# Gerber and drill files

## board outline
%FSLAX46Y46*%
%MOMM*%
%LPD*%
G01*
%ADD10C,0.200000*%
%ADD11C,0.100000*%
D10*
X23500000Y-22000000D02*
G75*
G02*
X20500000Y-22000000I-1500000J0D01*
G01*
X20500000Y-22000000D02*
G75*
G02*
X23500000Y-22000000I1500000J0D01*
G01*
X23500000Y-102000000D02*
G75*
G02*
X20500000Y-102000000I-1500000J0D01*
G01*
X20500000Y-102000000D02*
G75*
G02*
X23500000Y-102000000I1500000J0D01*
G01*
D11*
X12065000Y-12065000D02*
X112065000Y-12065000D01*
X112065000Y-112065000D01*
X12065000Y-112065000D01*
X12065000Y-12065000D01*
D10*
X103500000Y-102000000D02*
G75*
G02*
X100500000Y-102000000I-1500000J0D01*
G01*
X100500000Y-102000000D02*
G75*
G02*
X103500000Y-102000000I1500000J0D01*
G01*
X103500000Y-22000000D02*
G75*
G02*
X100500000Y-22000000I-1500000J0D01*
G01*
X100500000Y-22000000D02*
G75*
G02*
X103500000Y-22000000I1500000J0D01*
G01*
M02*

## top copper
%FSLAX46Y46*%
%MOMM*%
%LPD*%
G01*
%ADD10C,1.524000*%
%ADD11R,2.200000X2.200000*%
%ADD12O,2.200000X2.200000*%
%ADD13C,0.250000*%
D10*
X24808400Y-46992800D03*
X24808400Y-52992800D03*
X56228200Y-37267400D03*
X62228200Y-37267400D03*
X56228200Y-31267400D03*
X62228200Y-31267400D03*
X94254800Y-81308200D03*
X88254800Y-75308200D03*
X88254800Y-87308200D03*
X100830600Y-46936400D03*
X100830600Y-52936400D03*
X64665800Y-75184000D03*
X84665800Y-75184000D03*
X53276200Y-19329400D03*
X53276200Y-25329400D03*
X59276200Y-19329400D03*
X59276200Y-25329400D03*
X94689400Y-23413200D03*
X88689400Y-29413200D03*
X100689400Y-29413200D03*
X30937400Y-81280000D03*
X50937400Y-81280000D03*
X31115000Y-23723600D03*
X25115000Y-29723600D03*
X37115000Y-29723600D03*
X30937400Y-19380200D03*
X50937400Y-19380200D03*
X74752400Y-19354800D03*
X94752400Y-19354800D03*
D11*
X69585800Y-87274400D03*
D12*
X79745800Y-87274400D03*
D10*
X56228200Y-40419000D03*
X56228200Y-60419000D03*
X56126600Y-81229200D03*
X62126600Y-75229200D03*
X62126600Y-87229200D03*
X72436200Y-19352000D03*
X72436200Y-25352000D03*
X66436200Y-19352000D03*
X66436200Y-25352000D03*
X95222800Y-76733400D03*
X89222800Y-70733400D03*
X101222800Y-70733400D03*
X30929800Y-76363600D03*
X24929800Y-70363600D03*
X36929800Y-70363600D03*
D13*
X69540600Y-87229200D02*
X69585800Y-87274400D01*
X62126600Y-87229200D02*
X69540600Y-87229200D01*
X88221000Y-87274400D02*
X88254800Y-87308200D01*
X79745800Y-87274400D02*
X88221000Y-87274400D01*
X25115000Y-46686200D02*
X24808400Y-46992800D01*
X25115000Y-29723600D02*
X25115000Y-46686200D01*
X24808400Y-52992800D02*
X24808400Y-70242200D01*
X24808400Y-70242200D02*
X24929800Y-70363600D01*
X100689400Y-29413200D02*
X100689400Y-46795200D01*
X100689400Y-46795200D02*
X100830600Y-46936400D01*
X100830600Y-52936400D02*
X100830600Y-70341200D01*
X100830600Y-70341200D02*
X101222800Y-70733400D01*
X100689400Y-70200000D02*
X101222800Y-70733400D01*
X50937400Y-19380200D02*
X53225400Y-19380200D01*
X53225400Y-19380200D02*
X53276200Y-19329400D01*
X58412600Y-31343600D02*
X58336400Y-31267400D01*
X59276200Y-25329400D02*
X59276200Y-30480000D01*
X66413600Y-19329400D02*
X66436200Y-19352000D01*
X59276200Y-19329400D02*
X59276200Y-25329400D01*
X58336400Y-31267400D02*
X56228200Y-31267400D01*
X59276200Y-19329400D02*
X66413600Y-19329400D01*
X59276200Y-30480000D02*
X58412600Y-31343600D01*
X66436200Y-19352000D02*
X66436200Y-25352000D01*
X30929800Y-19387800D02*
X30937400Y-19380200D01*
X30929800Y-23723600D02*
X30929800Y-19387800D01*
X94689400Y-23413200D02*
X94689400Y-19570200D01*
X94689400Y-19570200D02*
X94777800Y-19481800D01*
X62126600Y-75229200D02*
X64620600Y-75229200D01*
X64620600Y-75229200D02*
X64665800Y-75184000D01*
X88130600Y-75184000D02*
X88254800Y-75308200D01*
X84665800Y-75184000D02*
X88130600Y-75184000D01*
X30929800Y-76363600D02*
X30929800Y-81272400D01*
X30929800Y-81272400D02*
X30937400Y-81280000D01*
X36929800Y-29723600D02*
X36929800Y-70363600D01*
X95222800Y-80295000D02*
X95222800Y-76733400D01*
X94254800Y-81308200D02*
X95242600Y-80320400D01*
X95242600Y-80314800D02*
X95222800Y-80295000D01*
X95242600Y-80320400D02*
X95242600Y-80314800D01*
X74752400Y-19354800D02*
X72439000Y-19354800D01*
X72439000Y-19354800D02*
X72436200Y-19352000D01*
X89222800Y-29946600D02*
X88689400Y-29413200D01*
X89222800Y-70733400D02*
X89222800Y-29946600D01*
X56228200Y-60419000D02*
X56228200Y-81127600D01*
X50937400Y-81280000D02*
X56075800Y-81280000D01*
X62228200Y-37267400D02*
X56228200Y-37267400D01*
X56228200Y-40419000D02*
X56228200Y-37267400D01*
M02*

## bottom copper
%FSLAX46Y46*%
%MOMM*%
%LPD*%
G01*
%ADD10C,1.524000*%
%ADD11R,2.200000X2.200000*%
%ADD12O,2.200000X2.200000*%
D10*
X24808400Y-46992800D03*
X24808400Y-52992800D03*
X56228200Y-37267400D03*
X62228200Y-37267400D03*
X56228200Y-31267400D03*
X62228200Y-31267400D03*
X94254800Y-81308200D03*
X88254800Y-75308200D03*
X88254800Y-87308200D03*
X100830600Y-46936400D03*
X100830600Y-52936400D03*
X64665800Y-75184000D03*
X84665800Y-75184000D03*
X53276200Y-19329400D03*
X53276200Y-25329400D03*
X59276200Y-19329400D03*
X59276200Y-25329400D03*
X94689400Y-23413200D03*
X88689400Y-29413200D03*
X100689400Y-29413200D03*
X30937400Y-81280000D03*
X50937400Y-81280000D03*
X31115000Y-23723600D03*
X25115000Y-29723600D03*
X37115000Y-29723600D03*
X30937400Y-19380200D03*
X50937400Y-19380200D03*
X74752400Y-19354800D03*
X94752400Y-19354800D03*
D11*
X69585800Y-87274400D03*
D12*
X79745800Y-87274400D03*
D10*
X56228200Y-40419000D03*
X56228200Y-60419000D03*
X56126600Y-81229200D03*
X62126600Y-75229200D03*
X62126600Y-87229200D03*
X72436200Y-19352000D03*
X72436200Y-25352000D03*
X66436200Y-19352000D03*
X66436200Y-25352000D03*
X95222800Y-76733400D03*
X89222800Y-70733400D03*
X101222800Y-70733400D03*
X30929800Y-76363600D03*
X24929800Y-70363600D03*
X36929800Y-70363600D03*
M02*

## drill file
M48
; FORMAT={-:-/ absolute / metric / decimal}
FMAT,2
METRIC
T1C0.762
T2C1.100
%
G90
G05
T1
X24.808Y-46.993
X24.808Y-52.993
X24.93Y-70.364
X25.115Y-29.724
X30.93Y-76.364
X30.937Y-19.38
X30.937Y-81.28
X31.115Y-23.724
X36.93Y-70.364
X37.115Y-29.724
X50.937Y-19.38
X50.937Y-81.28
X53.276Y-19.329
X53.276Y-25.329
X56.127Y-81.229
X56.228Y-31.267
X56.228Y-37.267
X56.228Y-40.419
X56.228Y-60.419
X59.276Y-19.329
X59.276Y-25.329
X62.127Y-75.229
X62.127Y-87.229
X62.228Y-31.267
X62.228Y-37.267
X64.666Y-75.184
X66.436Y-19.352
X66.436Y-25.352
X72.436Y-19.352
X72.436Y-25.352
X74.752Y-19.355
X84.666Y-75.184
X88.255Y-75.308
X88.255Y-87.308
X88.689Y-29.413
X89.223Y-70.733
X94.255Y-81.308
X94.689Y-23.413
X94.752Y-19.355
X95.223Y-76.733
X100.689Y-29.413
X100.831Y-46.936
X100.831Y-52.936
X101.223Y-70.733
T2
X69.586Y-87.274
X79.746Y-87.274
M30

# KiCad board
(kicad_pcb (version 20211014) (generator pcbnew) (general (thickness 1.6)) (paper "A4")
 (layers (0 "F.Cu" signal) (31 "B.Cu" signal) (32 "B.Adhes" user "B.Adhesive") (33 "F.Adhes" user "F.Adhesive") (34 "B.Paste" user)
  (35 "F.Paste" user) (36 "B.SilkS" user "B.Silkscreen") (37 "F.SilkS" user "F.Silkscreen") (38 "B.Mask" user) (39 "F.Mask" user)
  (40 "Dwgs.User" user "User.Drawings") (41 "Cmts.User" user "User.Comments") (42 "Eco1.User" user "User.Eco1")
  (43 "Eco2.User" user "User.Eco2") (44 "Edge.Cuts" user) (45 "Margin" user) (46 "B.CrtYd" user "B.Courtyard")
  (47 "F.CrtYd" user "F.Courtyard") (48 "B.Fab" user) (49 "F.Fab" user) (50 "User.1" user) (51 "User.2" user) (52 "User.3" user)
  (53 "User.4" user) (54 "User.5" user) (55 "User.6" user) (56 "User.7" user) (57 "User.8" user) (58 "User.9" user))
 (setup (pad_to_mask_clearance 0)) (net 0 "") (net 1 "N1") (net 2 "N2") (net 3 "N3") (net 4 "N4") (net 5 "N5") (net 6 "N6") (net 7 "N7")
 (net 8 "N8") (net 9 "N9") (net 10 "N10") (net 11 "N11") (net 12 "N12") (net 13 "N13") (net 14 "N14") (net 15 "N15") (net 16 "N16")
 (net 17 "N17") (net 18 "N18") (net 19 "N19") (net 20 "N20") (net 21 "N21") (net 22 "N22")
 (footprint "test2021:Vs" (layer "F.Cu") (at 24.8084 49.9928)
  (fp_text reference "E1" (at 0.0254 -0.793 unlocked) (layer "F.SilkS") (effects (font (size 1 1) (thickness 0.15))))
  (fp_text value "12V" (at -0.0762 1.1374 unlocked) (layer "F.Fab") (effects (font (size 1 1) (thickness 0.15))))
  (pad "1" thru_hole circle (at 0 -3) (size 1.524 1.524) (drill 0.762) (layers *.Cu *.Mask) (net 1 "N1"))
  (pad "2" thru_hole circle (at 0 3) (size 1.524 1.524) (drill 0.762) (layers *.Cu *.Mask) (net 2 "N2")))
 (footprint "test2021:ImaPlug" (layer "F.Cu") (at 59.2282 34.2674 90)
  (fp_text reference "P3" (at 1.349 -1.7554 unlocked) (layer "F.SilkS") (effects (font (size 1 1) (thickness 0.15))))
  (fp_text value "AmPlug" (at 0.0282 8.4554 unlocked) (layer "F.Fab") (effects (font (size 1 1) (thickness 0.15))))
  (pad "1" thru_hole circle (at -3 -3 90) (size 1.524 1.524) (drill 0.762) (layers *.Cu *.Mask) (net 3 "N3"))
  (pad "2" thru_hole circle (at -3 3 90) (size 1.524 1.524) (drill 0.762) (layers *.Cu *.Mask) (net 3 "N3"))
  (pad "3" thru_hole circle (at 3 -3 90) (size 1.524 1.524) (drill 0.762) (layers *.Cu *.Mask) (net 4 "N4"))
  (pad "4" thru_hole circle (at 3 3 90) (size 1.524 1.524) (drill 0.762) (layers *.Cu *.Mask) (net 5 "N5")))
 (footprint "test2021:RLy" (layer "F.Cu") (at 88.2548 81.3082 -90)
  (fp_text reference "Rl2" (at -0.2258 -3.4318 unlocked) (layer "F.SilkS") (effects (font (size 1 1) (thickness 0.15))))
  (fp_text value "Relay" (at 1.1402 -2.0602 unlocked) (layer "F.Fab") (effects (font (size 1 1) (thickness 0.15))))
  (pad "1" thru_hole circle (at 0 -6 270) (size 1.524 1.524) (drill 0.762) (layers *.Cu *.Mask) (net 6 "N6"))
  (pad "2" thru_hole circle (at -6 0 270) (size 1.524 1.524) (drill 0.762) (layers *.Cu *.Mask) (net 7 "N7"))
  (pad "3" thru_hole circle (at 6 0 270) (size 1.524 1.524) (drill 0.762) (layers *.Cu *.Mask) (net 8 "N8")))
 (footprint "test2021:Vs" (layer "F.Cu") (at 100.8306 49.9364)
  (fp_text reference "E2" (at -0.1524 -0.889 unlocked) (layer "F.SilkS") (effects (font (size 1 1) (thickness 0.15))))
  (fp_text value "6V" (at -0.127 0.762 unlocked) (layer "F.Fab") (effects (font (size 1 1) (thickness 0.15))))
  (pad "1" thru_hole circle (at 0 -3) (size 1.524 1.524) (drill 0.762) (layers *.Cu *.Mask) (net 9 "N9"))
  (pad "2" thru_hole circle (at 0 3) (size 1.524 1.524) (drill 0.762) (layers *.Cu *.Mask) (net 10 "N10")))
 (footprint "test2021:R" (layer "F.Cu") (at 74.6658 75.184)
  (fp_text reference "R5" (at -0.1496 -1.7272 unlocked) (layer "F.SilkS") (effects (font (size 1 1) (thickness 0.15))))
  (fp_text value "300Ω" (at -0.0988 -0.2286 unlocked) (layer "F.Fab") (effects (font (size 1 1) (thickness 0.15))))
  (pad "1" thru_hole circle (at -10 0) (size 1.524 1.524) (drill 0.762) (layers *.Cu *.Mask) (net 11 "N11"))
  (pad "2" thru_hole circle (at 10 0) (size 1.524 1.524) (drill 0.762) (layers *.Cu *.Mask) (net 7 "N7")))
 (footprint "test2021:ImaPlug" (layer "F.Cu") (at 56.2762 22.3294)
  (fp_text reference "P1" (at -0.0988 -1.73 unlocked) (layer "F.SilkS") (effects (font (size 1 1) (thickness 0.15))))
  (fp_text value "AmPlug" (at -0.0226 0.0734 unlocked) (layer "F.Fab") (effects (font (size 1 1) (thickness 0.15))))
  (pad "1" thru_hole circle (at -3 -3) (size 1.524 1.524) (drill 0.762) (layers *.Cu *.Mask) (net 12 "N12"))
  (pad "2" thru_hole circle (at -3 3) (size 1.524 1.524) (drill 0.762) (layers *.Cu *.Mask) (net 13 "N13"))
  (pad "3" thru_hole circle (at 3 -3) (size 1.524 1.524) (drill 0.762) (layers *.Cu *.Mask) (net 4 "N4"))
  (pad "4" thru_hole circle (at 3 3) (size 1.524 1.524) (drill 0.762) (layers *.Cu *.Mask) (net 4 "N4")))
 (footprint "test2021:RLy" (layer "F.Cu") (at 94.6894 29.4132)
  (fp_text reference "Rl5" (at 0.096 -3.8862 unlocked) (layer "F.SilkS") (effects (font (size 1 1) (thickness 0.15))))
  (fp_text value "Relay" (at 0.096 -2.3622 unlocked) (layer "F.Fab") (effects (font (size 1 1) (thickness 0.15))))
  (pad "1" thru_hole circle (at 0 -6) (size 1.524 1.524) (drill 0.762) (layers *.Cu *.Mask) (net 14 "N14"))
  (pad "2" thru_hole circle (at -6 0) (size 1.524 1.524) (drill 0.762) (layers *.Cu *.Mask) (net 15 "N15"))
  (pad "3" thru_hole circle (at 6 0) (size 1.524 1.524) (drill 0.762) (layers *.Cu *.Mask) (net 9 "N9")))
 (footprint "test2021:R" (layer "F.Cu") (at 40.9374 81.28)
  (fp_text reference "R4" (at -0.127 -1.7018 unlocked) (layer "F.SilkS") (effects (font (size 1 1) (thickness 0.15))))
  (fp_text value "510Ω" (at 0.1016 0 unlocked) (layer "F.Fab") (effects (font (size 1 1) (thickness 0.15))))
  (pad "1" thru_hole circle (at -10 0) (size 1.524 1.524) (drill 0.762) (layers *.Cu *.Mask) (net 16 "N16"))
  (pad "2" thru_hole circle (at 10 0) (size 1.524 1.524) (drill 0.762) (layers *.Cu *.Mask) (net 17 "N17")))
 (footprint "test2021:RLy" (layer "F.Cu") (at 31.115 29.7236)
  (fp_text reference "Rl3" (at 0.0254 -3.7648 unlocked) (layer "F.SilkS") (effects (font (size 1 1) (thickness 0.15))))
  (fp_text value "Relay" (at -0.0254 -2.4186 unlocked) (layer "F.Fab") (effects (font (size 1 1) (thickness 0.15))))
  (pad "1" thru_hole circle (at 0 -6) (size 1.524 1.524) (drill 0.762) (layers *.Cu *.Mask) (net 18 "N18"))
  (pad "2" thru_hole circle (at -6 0) (size 1.524 1.524) (drill 0.762) (layers *.Cu *.Mask) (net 1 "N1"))
  (pad "3" thru_hole circle (at 6 0) (size 1.524 1.524) (drill 0.762) (layers *.Cu *.Mask) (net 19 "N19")))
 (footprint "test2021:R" (layer "F.Cu") (at 40.9374 19.3802)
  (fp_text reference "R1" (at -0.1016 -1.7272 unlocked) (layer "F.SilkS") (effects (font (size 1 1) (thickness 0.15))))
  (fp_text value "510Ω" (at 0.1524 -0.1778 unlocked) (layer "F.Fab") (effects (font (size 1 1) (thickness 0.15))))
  (pad "1" thru_hole circle (at -10 0) (size 1.524 1.524) (drill 0.762) (layers *.Cu *.Mask) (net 18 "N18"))
  (pad "2" thru_hole circle (at 10 0) (size 1.524 1.524) (drill 0.762) (layers *.Cu *.Mask) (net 12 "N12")))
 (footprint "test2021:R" (layer "F.Cu") (at 84.7524 19.3548)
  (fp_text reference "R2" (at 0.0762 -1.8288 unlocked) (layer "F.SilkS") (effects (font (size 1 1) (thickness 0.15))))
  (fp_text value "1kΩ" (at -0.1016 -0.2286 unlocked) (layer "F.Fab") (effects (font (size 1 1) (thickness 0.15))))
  (pad "1" thru_hole circle (at -10 0) (size 1.524 1.524) (drill 0.762) (layers *.Cu *.Mask) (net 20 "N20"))
  (pad "2" thru_hole circle (at 10 0) (size 1.524 1.524) (drill 0.762) (layers *.Cu *.Mask) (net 14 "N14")))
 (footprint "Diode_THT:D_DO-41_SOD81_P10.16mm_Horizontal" (layer "F.Cu") (at 69.5858 87.2744)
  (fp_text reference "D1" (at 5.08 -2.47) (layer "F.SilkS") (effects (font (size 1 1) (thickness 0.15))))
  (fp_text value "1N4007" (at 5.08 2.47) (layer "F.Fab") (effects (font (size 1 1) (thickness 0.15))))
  (pad "1" thru_hole rect (at 0 0) (size 2.2 2.2) (drill 1.1) (layers *.Cu *.Mask) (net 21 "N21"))
  (pad "2" thru_hole oval (at 10.16 0) (size 2.2 2.2) (drill 1.1) (layers *.Cu *.Mask) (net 8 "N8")))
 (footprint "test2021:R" (layer "F.Cu") (at 56.2282 50.419 -90)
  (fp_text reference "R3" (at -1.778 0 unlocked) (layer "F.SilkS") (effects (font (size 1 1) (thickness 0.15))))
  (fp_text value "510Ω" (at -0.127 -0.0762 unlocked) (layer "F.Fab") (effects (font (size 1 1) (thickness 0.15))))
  (pad "1" thru_hole circle (at -10 0 270) (size 1.524 1.524) (drill 0.762) (layers *.Cu *.Mask) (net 3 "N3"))
  (pad "2" thru_hole circle (at 10 0 270) (size 1.524 1.524) (drill 0.762) (layers *.Cu *.Mask) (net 17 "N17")))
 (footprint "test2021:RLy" (layer "B.Cu") (at 62.1266 81.2292 -90)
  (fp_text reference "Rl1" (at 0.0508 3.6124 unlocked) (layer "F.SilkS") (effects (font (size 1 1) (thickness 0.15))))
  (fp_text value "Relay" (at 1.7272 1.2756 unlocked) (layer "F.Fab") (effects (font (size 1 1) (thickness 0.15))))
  (pad "1" thru_hole circle (at 0 6 270) (size 1.524 1.524) (drill 0.762) (layers *.Cu *.Mask) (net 17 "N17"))
  (pad "2" thru_hole circle (at -6 0 270) (size 1.524 1.524) (drill 0.762) (layers *.Cu *.Mask) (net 11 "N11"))
  (pad "3" thru_hole circle (at 6 0 270) (size 1.524 1.524) (drill 0.762) (layers *.Cu *.Mask) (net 21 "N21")))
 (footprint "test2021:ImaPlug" (layer "B.Cu") (at 69.4362 22.352 180)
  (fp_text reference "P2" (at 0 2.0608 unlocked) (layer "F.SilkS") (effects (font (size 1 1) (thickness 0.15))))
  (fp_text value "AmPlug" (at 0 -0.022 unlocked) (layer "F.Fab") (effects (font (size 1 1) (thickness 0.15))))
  (pad "1" thru_hole circle (at -3 3 180) (size 1.524 1.524) (drill 0.762) (layers *.Cu *.Mask) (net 20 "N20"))
  (pad "2" thru_hole circle (at -3 -3 180) (size 1.524 1.524) (drill 0.762) (layers *.Cu *.Mask) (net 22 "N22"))
  (pad "3" thru_hole circle (at 3 3 180) (size 1.524 1.524) (drill 0.762) (layers *.Cu *.Mask) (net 4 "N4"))
  (pad "4" thru_hole circle (at 3 -3 180) (size 1.524 1.524) (drill 0.762) (layers *.Cu *.Mask) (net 4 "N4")))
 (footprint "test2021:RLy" (layer "B.Cu") (at 95.2228 70.7334)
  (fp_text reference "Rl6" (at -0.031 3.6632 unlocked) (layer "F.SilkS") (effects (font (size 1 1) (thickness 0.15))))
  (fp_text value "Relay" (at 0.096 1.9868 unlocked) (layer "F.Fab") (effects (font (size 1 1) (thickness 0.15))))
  (pad "1" thru_hole circle (at 0 6) (size 1.524 1.524) (drill 0.762) (layers *.Cu *.Mask) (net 6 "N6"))
  (pad "2" thru_hole circle (at -6 0) (size 1.524 1.524) (drill 0.762) (layers *.Cu *.Mask) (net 15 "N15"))
  (pad "3" thru_hole circle (at 6 0) (size 1.524 1.524) (drill 0.762) (layers *.Cu *.Mask) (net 10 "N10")))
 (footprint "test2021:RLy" (layer "B.Cu") (at 30.9298 70.3636)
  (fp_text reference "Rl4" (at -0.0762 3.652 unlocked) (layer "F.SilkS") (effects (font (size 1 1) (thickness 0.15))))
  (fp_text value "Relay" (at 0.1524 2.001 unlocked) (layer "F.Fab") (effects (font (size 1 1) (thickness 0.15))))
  (pad "1" thru_hole circle (at 0 6) (size 1.524 1.524) (drill 0.762) (layers *.Cu *.Mask) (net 16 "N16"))
  (pad "2" thru_hole circle (at -6 0) (size 1.524 1.524) (drill 0.762) (layers *.Cu *.Mask) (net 2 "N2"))
  (pad "3" thru_hole circle (at 6 0) (size 1.524 1.524) (drill 0.762) (layers *.Cu *.Mask) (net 19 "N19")))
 (gr_circle (center 22 22) (end 23.5 22) (layer "Edge.Cuts") (width 0.2) (fill none))
 (gr_circle (center 22 102) (end 23.5 102) (layer "Edge.Cuts") (width 0.2) (fill none))
 (gr_rect (start 12.065 12.065) (end 112.065 112.065) (layer "Edge.Cuts") (width 0.1) (fill none))
 (gr_circle (center 102 102) (end 103.5 102) (layer "Edge.Cuts") (width 0.2) (fill none))
 (gr_circle (center 102 22) (end 103.5 22) (layer "Edge.Cuts") (width 0.2) (fill none))
 (segment (start 69.5406 87.2292) (end 69.5858 87.2744) (width 0.25) (layer "F.Cu") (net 21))
 (segment (start 62.1266 87.2292) (end 69.5406 87.2292) (width 0.25) (layer "F.Cu") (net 21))
 (segment (start 88.221 87.2744) (end 88.2548 87.3082) (width 0.25) (layer "F.Cu") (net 8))
 (segment (start 79.7458 87.2744) (end 88.221 87.2744) (width 0.25) (layer "F.Cu") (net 8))
 (segment (start 25.115 46.6862) (end 24.8084 46.9928) (width 0.25) (layer "F.Cu") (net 1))
 (segment (start 25.115 29.7236) (end 25.115 46.6862) (width 0.25) (layer "F.Cu") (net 1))
 (segment (start 24.8084 52.9928) (end 24.8084 70.2422) (width 0.25) (layer "F.Cu") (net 2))
 (segment (start 24.8084 70.2422) (end 24.9298 70.3636) (width 0.25) (layer "F.Cu") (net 2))
 (segment (start 100.6894 29.4132) (end 100.6894 46.7952) (width 0.25) (layer "F.Cu") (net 9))
 (segment (start 100.6894 46.7952) (end 100.8306 46.9364) (width 0.25) (layer "F.Cu") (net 9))
 (segment (start 100.8306 52.9364) (end 100.8306 70.3412) (width 0.25) (layer "F.Cu") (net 10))
 (segment (start 100.8306 70.3412) (end 101.2228 70.7334) (width 0.25) (layer "F.Cu") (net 10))
 (segment (start 100.6894 70.2) (end 101.2228 70.7334) (width 0.25) (layer "F.Cu") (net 10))
 (segment (start 50.9374 19.3802) (end 53.2254 19.3802) (width 0.25) (layer "F.Cu") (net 12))
 (segment (start 53.2254 19.3802) (end 53.2762 19.3294) (width 0.25) (layer "F.Cu") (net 12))
 (segment (start 58.4126 31.3436) (end 58.3364 31.2674) (width 0.25) (layer "F.Cu") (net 4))
 (segment (start 59.2762 25.3294) (end 59.2762 30.48) (width 0.25) (layer "F.Cu") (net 4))
 (segment (start 66.4136 19.3294) (end 66.4362 19.352) (width 0.25) (layer "F.Cu") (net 4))
 (segment (start 59.2762 19.3294) (end 59.2762 25.3294) (width 0.25) (layer "F.Cu") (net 4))
 (segment (start 58.3364 31.2674) (end 56.2282 31.2674) (width 0.25) (layer "F.Cu") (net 4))
 (segment (start 59.2762 19.3294) (end 66.4136 19.3294) (width 0.25) (layer "F.Cu") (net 4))
 (segment (start 59.2762 30.48) (end 58.4126 31.3436) (width 0.25) (layer "F.Cu") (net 4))
 (segment (start 66.4362 19.352) (end 66.4362 25.352) (width 0.25) (layer "F.Cu") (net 4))
 (segment (start 30.9298 19.3878) (end 30.9374 19.3802) (width 0.25) (layer "F.Cu") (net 18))
 (segment (start 30.9298 23.7236) (end 30.9298 19.3878) (width 0.25) (layer "F.Cu") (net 18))
 (segment (start 94.6894 23.4132) (end 94.6894 19.5702) (width 0.25) (layer "F.Cu") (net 14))
 (segment (start 94.6894 19.5702) (end 94.7778 19.4818) (width 0.25) (layer "F.Cu") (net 14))
 (segment (start 62.1266 75.2292) (end 64.6206 75.2292) (width 0.25) (layer "F.Cu") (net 11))
 (segment (start 64.6206 75.2292) (end 64.6658 75.184) (width 0.25) (layer "F.Cu") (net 11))
 (segment (start 88.1306 75.184) (end 88.2548 75.3082) (width 0.25) (layer "F.Cu") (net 7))
 (segment (start 84.6658 75.184) (end 88.1306 75.184) (width 0.25) (layer "F.Cu") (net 7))
 (segment (start 30.9298 76.3636) (end 30.9298 81.2724) (width 0.25) (layer "F.Cu") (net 16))
 (segment (start 30.9298 81.2724) (end 30.9374 81.28) (width 0.25) (layer "F.Cu") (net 16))
 (segment (start 36.9298 29.7236) (end 36.9298 70.3636) (width 0.25) (layer "F.Cu") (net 19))
 (segment (start 95.2228 80.295) (end 95.2228 76.7334) (width 0.25) (layer "F.Cu") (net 6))
 (segment (start 94.2548 81.3082) (end 95.2426 80.3204) (width 0.25) (layer "F.Cu") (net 6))
 (segment (start 95.2426 80.3148) (end 95.2228 80.295) (width 0.25) (layer "F.Cu") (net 6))
 (segment (start 95.2426 80.3204) (end 95.2426 80.3148) (width 0.25) (layer "F.Cu") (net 6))
 (segment (start 74.7524 19.3548) (end 72.439 19.3548) (width 0.25) (layer "F.Cu") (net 20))
 (segment (start 72.439 19.3548) (end 72.4362 19.352) (width 0.25) (layer "F.Cu") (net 20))
 (segment (start 89.2228 29.9466) (end 88.6894 29.4132) (width 0.25) (layer "F.Cu") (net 15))
 (segment (start 89.2228 70.7334) (end 89.2228 29.9466) (width 0.25) (layer "F.Cu") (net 15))
 (segment (start 56.2282 60.419) (end 56.2282 81.1276) (width 0.25) (layer "F.Cu") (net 17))
 (segment (start 50.9374 81.28) (end 56.0758 81.28) (width 0.25) (layer "F.Cu") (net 17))
 (segment (start 62.2282 37.2674) (end 56.2282 37.2674) (width 0.25) (layer "F.Cu") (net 3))
 (segment (start 56.2282 40.419) (end 56.2282 37.2674) (width 0.25) (layer "F.Cu") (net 3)))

